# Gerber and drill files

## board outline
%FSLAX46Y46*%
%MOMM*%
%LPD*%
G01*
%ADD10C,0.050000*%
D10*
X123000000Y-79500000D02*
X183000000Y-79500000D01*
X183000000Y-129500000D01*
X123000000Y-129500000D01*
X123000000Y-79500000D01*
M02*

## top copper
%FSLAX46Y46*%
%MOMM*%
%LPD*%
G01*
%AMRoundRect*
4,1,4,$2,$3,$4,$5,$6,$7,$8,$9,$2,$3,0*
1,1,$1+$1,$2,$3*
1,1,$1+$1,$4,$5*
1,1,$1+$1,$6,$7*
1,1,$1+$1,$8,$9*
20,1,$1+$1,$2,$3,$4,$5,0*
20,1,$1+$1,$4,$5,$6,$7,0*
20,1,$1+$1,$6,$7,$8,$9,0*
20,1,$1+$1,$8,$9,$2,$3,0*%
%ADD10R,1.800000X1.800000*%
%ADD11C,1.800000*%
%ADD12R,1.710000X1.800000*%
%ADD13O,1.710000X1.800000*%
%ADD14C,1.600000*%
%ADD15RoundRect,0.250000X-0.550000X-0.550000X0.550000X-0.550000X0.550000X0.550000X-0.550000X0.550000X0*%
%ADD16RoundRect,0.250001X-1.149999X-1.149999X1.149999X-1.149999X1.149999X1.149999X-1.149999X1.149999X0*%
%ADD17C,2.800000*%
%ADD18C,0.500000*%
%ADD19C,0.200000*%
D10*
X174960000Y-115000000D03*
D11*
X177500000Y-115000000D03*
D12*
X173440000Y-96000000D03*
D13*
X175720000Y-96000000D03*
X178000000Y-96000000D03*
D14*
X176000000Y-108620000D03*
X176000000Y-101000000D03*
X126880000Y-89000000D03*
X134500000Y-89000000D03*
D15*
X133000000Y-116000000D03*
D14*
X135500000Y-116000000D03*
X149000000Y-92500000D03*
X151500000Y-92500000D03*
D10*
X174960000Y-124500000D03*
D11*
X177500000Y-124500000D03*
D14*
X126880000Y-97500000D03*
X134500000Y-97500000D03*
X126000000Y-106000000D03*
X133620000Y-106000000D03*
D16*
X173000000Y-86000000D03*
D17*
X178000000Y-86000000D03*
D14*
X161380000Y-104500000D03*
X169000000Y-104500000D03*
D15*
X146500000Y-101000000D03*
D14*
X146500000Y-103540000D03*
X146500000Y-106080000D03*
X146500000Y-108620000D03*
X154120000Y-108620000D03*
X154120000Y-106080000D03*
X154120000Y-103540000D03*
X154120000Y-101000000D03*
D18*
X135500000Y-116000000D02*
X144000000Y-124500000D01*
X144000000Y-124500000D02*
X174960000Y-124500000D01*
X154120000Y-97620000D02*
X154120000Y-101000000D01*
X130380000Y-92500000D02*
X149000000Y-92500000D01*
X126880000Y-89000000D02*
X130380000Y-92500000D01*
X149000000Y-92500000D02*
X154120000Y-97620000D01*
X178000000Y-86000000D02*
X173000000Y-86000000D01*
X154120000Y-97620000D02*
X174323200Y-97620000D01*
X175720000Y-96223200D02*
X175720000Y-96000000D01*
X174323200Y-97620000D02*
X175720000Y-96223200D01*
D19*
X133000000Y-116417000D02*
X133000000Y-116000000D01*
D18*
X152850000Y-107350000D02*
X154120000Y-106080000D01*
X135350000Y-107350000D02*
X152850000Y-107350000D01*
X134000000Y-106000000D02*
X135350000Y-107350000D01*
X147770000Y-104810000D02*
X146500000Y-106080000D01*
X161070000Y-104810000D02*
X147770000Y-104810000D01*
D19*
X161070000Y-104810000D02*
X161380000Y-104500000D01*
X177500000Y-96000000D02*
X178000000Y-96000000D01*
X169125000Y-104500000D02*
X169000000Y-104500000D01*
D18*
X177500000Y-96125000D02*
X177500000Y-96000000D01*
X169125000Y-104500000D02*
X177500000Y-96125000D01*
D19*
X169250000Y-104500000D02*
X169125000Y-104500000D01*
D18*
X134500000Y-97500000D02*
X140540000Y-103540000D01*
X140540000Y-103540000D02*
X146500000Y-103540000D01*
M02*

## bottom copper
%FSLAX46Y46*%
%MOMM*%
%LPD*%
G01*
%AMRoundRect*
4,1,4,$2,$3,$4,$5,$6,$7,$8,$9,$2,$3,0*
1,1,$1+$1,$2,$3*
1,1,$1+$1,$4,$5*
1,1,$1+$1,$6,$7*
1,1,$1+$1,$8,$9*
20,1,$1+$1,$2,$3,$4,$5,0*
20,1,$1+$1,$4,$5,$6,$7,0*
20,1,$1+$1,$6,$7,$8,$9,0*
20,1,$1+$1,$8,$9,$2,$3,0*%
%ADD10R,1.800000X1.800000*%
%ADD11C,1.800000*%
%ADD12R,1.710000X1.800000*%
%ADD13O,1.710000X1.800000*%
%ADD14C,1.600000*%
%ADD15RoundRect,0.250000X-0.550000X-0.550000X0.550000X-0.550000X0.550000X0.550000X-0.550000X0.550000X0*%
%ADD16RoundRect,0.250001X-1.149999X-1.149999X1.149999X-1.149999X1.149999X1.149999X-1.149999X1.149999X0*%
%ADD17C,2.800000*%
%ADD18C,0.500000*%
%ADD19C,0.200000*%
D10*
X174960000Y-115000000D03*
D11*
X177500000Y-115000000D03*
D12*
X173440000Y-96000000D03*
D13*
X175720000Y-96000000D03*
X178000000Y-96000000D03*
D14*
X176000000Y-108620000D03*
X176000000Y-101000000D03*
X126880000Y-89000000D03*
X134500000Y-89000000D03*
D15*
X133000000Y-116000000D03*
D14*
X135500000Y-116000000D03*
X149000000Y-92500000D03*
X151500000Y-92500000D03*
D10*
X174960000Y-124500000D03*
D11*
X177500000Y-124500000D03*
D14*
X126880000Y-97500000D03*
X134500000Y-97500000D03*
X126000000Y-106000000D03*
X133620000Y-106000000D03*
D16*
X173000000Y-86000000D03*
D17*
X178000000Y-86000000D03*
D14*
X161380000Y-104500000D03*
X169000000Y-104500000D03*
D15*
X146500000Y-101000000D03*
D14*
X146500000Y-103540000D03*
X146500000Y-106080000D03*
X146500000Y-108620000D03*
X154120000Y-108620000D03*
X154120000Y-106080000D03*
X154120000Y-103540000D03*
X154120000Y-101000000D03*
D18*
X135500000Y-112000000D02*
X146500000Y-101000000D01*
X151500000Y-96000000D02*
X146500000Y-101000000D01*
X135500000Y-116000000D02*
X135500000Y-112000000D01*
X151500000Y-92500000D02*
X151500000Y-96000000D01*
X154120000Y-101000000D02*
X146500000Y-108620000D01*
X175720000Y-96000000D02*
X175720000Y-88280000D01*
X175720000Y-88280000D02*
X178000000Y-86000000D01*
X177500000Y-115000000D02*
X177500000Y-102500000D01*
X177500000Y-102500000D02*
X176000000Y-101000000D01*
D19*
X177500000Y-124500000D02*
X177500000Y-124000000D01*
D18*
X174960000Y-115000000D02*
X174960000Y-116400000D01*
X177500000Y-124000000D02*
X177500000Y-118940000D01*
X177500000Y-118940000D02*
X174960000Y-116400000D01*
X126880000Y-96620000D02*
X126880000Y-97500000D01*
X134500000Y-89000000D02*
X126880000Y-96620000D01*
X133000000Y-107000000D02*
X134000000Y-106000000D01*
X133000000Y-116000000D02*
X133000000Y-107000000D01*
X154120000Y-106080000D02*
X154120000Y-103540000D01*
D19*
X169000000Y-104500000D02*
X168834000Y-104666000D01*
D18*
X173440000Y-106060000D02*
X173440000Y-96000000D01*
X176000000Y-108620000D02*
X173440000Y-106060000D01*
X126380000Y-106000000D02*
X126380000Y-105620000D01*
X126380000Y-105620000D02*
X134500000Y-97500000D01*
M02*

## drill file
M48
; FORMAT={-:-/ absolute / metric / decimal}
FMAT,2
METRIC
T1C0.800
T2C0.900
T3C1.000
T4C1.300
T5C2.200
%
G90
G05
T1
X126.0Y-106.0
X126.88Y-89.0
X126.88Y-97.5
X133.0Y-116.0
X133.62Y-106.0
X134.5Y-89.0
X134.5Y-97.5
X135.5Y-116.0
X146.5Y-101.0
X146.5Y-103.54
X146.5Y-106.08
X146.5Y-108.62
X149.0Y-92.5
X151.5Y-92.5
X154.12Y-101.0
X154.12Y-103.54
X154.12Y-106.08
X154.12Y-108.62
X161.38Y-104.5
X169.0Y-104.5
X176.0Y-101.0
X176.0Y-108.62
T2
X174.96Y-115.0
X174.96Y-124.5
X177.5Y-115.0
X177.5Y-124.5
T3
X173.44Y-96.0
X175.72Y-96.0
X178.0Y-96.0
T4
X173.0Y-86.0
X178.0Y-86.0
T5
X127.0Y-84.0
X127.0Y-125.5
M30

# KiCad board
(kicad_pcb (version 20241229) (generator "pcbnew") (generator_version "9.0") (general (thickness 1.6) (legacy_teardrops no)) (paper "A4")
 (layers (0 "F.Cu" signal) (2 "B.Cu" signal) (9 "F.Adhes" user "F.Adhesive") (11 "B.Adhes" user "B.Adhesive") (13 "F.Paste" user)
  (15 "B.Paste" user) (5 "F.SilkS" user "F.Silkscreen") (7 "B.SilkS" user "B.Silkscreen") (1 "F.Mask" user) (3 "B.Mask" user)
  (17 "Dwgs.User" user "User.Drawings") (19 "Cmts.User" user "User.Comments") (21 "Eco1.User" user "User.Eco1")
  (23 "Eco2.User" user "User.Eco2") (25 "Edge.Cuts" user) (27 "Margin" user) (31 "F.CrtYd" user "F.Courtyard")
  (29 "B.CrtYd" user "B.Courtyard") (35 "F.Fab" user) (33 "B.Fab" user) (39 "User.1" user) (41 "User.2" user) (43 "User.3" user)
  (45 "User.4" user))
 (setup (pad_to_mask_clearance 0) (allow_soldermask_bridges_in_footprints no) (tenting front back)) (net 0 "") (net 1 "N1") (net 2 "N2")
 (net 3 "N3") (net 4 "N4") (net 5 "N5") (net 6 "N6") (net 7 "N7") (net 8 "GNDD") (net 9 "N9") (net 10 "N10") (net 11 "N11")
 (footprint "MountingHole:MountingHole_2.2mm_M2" (layer "F.Cu") (at 127 84)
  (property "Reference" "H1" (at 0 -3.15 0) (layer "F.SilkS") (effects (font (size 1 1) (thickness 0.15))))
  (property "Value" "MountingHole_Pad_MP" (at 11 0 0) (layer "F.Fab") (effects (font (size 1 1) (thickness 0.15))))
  (pad "" np_thru_hole circle (at 0 0) (size 2.2 2.2) (drill 2.2) (layers "*.Cu" "*.Mask")))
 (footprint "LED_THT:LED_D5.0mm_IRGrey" (layer "F.Cu") (at 174.96 115)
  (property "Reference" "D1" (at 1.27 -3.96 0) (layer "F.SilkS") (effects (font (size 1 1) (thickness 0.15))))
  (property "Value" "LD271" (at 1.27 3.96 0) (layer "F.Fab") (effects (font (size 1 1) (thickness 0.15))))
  (pad "1" thru_hole rect (at 0 0) (size 1.8 1.8) (drill 0.9) (layers "*.Cu" "*.Mask") (remove_unused_layers no) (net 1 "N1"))
  (pad "2" thru_hole circle (at 2.54 0) (size 1.8 1.8) (drill 0.9) (layers "*.Cu" "*.Mask") (remove_unused_layers no) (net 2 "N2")))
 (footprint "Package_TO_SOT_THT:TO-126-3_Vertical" (layer "F.Cu") (at 173.44 96)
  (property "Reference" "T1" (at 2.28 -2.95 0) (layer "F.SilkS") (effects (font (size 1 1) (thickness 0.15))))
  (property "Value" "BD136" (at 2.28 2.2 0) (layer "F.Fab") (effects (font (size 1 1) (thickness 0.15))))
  (pad "1" thru_hole rect (at 0 0) (size 1.71 1.8) (drill 1) (layers "*.Cu" "*.Mask") (remove_unused_layers no) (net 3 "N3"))
  (pad "2" thru_hole oval (at 2.28 0) (size 1.71 1.8) (drill 1) (layers "*.Cu" "*.Mask") (remove_unused_layers no) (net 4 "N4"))
  (pad "3" thru_hole oval (at 4.56 0) (size 1.71 1.8) (drill 1) (layers "*.Cu" "*.Mask") (remove_unused_layers no) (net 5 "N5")))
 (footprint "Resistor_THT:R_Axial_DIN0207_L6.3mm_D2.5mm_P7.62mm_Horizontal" (layer "F.Cu") (at 176 108.62 90)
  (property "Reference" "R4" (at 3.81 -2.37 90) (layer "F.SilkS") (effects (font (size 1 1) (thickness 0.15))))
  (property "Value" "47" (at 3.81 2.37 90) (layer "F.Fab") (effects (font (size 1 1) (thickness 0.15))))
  (pad "1" thru_hole circle (at 0 0 90) (size 1.6 1.6) (drill 0.8) (layers "*.Cu" "*.Mask") (remove_unused_layers no) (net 3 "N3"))
  (pad "2" thru_hole circle (at 7.62 0 90) (size 1.6 1.6) (drill 0.8) (layers "*.Cu" "*.Mask") (remove_unused_layers no) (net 2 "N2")))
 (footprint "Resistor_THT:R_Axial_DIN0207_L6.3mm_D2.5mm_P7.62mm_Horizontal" (layer "F.Cu") (at 126.88 89)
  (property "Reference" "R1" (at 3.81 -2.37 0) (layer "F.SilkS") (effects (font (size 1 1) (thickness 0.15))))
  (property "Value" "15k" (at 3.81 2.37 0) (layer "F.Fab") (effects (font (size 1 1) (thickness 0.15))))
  (pad "1" thru_hole circle (at 0 0) (size 1.6 1.6) (drill 0.8) (layers "*.Cu" "*.Mask") (remove_unused_layers no) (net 4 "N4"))
  (pad "2" thru_hole circle (at 7.62 0) (size 1.6 1.6) (drill 0.8) (layers "*.Cu" "*.Mask") (remove_unused_layers no) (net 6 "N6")))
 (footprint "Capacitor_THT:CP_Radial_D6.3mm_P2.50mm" (layer "F.Cu") (at 133 116)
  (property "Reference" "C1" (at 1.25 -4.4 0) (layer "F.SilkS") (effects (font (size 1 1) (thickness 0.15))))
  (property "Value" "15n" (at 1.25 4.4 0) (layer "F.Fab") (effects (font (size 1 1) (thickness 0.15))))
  (pad "1" thru_hole roundrect (at 0 0) (size 1.6 1.6) (drill 0.8) (layers "*.Cu" "*.Mask") (remove_unused_layers no)
   (roundrect_rratio 0.15625) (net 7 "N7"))
  (pad "2" thru_hole circle (at 2.5 0) (size 1.6 1.6) (drill 0.8) (layers "*.Cu" "*.Mask") (remove_unused_layers no) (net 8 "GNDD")))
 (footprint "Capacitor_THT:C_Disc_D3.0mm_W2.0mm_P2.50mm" (layer "F.Cu") (at 149 92.5)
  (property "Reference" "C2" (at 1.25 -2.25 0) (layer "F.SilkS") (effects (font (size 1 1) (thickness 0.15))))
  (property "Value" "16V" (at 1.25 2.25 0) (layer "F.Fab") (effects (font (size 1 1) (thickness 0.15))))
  (pad "1" thru_hole circle (at 0 0) (size 1.6 1.6) (drill 0.8) (layers "*.Cu" "*.Mask") (remove_unused_layers no) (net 4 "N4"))
  (pad "2" thru_hole circle (at 2.5 0) (size 1.6 1.6) (drill 0.8) (layers "*.Cu" "*.Mask") (remove_unused_layers no) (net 8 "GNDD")))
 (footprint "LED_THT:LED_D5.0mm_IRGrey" (layer "F.Cu") (at 174.96 124.5)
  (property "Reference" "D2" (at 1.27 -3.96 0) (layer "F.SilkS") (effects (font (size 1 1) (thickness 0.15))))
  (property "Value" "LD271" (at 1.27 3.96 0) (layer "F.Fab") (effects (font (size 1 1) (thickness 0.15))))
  (pad "1" thru_hole rect (at 0 0) (size 1.8 1.8) (drill 0.9) (layers "*.Cu" "*.Mask") (remove_unused_layers no) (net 8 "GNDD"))
  (pad "2" thru_hole circle (at 2.54 0) (size 1.8 1.8) (drill 0.9) (layers "*.Cu" "*.Mask") (remove_unused_layers no) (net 1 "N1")))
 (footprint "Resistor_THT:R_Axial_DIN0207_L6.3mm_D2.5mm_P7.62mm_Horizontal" (layer "F.Cu") (at 126.88 97.5)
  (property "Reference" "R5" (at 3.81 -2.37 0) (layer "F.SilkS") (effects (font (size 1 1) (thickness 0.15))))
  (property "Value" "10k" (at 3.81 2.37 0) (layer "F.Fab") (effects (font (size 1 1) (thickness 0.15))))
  (pad "1" thru_hole circle (at 0 0) (size 1.6 1.6) (drill 0.8) (layers "*.Cu" "*.Mask") (remove_unused_layers no) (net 6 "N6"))
  (pad "2" thru_hole circle (at 7.62 0) (size 1.6 1.6) (drill 0.8) (layers "*.Cu" "*.Mask") (remove_unused_layers no) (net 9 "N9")))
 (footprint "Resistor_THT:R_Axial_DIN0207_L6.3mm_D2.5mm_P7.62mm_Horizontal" (layer "F.Cu") (at 126 106)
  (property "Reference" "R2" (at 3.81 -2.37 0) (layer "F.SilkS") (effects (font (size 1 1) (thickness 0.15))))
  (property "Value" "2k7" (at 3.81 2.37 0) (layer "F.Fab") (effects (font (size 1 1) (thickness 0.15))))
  (pad "1" thru_hole circle (at 0 0) (size 1.6 1.6) (drill 0.8) (layers "*.Cu" "*.Mask") (remove_unused_layers no) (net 9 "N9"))
  (pad "2" thru_hole circle (at 7.62 0) (size 1.6 1.6) (drill 0.8) (layers "*.Cu" "*.Mask") (remove_unused_layers no) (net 7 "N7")))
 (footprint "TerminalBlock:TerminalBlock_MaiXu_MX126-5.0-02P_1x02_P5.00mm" (layer "F.Cu") (at 173 86)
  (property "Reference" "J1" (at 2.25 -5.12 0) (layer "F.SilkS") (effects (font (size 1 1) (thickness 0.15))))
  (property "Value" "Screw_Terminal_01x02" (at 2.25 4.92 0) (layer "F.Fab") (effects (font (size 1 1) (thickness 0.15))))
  (pad "1" thru_hole roundrect (at 0 0) (size 2.8 2.8) (drill 1.3) (layers "*.Cu" "*.Mask") (remove_unused_layers no)
   (roundrect_rratio 0.089286) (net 4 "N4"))
  (pad "2" thru_hole circle (at 5 0) (size 2.8 2.8) (drill 1.3) (layers "*.Cu" "*.Mask") (remove_unused_layers no) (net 4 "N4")))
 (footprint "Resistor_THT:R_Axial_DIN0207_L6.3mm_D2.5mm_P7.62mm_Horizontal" (layer "F.Cu") (at 161.38 104.5)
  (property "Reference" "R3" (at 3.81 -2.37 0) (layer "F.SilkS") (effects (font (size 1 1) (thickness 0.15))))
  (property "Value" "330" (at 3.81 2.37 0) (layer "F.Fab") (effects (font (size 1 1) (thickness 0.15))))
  (pad "1" thru_hole circle (at 0 0) (size 1.6 1.6) (drill 0.8) (layers "*.Cu" "*.Mask") (remove_unused_layers no) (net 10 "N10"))
  (pad "2" thru_hole circle (at 7.62 0) (size 1.6 1.6) (drill 0.8) (layers "*.Cu" "*.Mask") (remove_unused_layers no) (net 5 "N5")))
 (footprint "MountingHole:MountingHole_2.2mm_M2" (layer "F.Cu") (at 127 125.5)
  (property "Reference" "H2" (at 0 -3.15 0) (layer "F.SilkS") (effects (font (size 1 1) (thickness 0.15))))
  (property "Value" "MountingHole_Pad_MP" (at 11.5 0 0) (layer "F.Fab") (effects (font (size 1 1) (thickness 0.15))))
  (pad "" np_thru_hole circle (at 0 0) (size 2.2 2.2) (drill 2.2) (layers "*.Cu" "*.Mask")))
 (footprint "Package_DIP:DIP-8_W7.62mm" (layer "F.Cu") (at 146.5 101)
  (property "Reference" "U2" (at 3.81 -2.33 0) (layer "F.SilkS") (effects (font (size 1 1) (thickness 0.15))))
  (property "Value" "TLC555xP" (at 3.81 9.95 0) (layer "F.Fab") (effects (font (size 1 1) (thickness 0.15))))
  (pad "1" thru_hole roundrect (at 0 0) (size 1.6 1.6) (drill 0.8) (layers "*.Cu" "*.Mask") (remove_unused_layers no)
   (roundrect_rratio 0.15625) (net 8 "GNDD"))
  (pad "2" thru_hole circle (at 0 2.54) (size 1.6 1.6) (drill 0.8) (layers "*.Cu" "*.Mask") (remove_unused_layers no) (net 9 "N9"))
  (pad "3" thru_hole circle (at 0 5.08) (size 1.6 1.6) (drill 0.8) (layers "*.Cu" "*.Mask") (remove_unused_layers no) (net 10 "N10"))
  (pad "4" thru_hole circle (at 0 7.62) (size 1.6 1.6) (drill 0.8) (layers "*.Cu" "*.Mask") (remove_unused_layers no) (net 4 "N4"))
  (pad "5" thru_hole circle (at 7.62 7.62) (size 1.6 1.6) (drill 0.8) (layers "*.Cu" "*.Mask") (remove_unused_layers no) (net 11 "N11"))
  (pad "6" thru_hole circle (at 7.62 5.08) (size 1.6 1.6) (drill 0.8) (layers "*.Cu" "*.Mask") (remove_unused_layers no) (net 7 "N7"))
  (pad "7" thru_hole circle (at 7.62 2.54) (size 1.6 1.6) (drill 0.8) (layers "*.Cu" "*.Mask") (remove_unused_layers no) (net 7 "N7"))
  (pad "8" thru_hole circle (at 7.62 0) (size 1.6 1.6) (drill 0.8) (layers "*.Cu" "*.Mask") (remove_unused_layers no) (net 4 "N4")))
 (gr_rect (start 123 79.5) (end 183 129.5) (stroke (width 0.05) (type solid)) (fill no) (layer "Edge.Cuts"))
 (segment (start 135.5 116) (end 144 124.5) (width 0.5) (layer "F.Cu") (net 8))
 (segment (start 144 124.5) (end 174.96 124.5) (width 0.5) (layer "F.Cu") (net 8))
 (segment (start 135.5 112) (end 146.5 101) (width 0.5) (layer "B.Cu") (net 8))
 (segment (start 151.5 96) (end 146.5 101) (width 0.5) (layer "B.Cu") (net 8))
 (segment (start 135.5 116) (end 135.5 112) (width 0.5) (layer "B.Cu") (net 8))
 (segment (start 151.5 92.5) (end 151.5 96) (width 0.5) (layer "B.Cu") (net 8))
 (segment (start 154.12 97.62) (end 154.12 101) (width 0.5) (layer "F.Cu") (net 4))
 (segment (start 130.38 92.5) (end 149 92.5) (width 0.5) (layer "F.Cu") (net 4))
 (segment (start 126.88 89) (end 130.38 92.5) (width 0.5) (layer "F.Cu") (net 4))
 (segment (start 149 92.5) (end 154.12 97.62) (width 0.5) (layer "F.Cu") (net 4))
 (segment (start 178 86) (end 173 86) (width 0.5) (layer "F.Cu") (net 4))
 (segment (start 154.12 97.62) (end 174.3232 97.62) (width 0.5) (layer "F.Cu") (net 4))
 (segment (start 175.72 96.2232) (end 175.72 96) (width 0.5) (layer "F.Cu") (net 4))
 (segment (start 174.3232 97.62) (end 175.72 96.2232) (width 0.5) (layer "F.Cu") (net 4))
 (segment (start 154.12 101) (end 146.5 108.62) (width 0.5) (layer "B.Cu") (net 4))
 (segment (start 175.72 96) (end 175.72 88.28) (width 0.5) (layer "B.Cu") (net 4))
 (segment (start 175.72 88.28) (end 178 86) (width 0.5) (layer "B.Cu") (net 4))
 (segment (start 177.5 115) (end 177.5 102.5) (width 0.5) (layer "B.Cu") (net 2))
 (segment (start 177.5 102.5) (end 176 101) (width 0.5) (layer "B.Cu") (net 2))
 (segment (start 177.5 124.5) (end 177.5 124) (width 0.2) (layer "B.Cu") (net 1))
 (segment (start 174.96 115) (end 174.96 116.4) (width 0.5) (layer "B.Cu") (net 1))
 (segment (start 177.5 124) (end 177.5 118.94) (width 0.5) (layer "B.Cu") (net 1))
 (segment (start 177.5 118.94) (end 174.96 116.4) (width 0.5) (layer "B.Cu") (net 1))
 (segment (start 126.88 96.62) (end 126.88 97.5) (width 0.5) (layer "B.Cu") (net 6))
 (segment (start 134.5 89) (end 126.88 96.62) (width 0.5) (layer "B.Cu") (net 6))
 (segment (start 133 116.417) (end 133 116) (width 0.2) (layer "F.Cu") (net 7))
 (segment (start 152.85 107.35) (end 154.12 106.08) (width 0.5) (layer "F.Cu") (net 7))
 (segment (start 135.35 107.35) (end 152.85 107.35) (width 0.5) (layer "F.Cu") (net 7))
 (segment (start 134 106) (end 135.35 107.35) (width 0.5) (layer "F.Cu") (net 7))
 (segment (start 133 107) (end 134 106) (width 0.5) (layer "B.Cu") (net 7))
 (segment (start 133 116) (end 133 107) (width 0.5) (layer "B.Cu") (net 7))
 (segment (start 154.12 106.08) (end 154.12 103.54) (width 0.5) (layer "B.Cu") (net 7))
 (segment (start 147.77 104.81) (end 146.5 106.08) (width 0.5) (layer "F.Cu") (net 10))
 (segment (start 161.07 104.81) (end 147.77 104.81) (width 0.5) (layer "F.Cu") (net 10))
 (segment (start 161.07 104.81) (end 161.38 104.5) (width 0.2) (layer "F.Cu") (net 10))
 (segment (start 177.5 96) (end 178 96) (width 0.2) (layer "F.Cu") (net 5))
 (segment (start 169.125 104.5) (end 169 104.5) (width 0.2) (layer "F.Cu") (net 5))
 (segment (start 177.5 96.125) (end 177.5 96) (width 0.5) (layer "F.Cu") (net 5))
 (segment (start 169.125 104.5) (end 177.5 96.125) (width 0.5) (layer "F.Cu") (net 5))
 (segment (start 169.25 104.5) (end 169.125 104.5) (width 0.2) (layer "F.Cu") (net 5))
 (segment (start 169 104.5) (end 168.834 104.666) (width 0.2) (layer "B.Cu") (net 5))
 (segment (start 173.44 106.06) (end 173.44 96) (width 0.5) (layer "B.Cu") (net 3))
 (segment (start 176 108.62) (end 173.44 106.06) (width 0.5) (layer "B.Cu") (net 3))
 (segment (start 134.5 97.5) (end 140.54 103.54) (width 0.5) (layer "F.Cu") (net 9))
 (segment (start 140.54 103.54) (end 146.5 103.54) (width 0.5) (layer "F.Cu") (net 9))
 (segment (start 126.38 106) (end 126.38 105.62) (width 0.5) (layer "B.Cu") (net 9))
 (segment (start 126.38 105.62) (end 134.5 97.5) (width 0.5) (layer "B.Cu") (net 9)))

